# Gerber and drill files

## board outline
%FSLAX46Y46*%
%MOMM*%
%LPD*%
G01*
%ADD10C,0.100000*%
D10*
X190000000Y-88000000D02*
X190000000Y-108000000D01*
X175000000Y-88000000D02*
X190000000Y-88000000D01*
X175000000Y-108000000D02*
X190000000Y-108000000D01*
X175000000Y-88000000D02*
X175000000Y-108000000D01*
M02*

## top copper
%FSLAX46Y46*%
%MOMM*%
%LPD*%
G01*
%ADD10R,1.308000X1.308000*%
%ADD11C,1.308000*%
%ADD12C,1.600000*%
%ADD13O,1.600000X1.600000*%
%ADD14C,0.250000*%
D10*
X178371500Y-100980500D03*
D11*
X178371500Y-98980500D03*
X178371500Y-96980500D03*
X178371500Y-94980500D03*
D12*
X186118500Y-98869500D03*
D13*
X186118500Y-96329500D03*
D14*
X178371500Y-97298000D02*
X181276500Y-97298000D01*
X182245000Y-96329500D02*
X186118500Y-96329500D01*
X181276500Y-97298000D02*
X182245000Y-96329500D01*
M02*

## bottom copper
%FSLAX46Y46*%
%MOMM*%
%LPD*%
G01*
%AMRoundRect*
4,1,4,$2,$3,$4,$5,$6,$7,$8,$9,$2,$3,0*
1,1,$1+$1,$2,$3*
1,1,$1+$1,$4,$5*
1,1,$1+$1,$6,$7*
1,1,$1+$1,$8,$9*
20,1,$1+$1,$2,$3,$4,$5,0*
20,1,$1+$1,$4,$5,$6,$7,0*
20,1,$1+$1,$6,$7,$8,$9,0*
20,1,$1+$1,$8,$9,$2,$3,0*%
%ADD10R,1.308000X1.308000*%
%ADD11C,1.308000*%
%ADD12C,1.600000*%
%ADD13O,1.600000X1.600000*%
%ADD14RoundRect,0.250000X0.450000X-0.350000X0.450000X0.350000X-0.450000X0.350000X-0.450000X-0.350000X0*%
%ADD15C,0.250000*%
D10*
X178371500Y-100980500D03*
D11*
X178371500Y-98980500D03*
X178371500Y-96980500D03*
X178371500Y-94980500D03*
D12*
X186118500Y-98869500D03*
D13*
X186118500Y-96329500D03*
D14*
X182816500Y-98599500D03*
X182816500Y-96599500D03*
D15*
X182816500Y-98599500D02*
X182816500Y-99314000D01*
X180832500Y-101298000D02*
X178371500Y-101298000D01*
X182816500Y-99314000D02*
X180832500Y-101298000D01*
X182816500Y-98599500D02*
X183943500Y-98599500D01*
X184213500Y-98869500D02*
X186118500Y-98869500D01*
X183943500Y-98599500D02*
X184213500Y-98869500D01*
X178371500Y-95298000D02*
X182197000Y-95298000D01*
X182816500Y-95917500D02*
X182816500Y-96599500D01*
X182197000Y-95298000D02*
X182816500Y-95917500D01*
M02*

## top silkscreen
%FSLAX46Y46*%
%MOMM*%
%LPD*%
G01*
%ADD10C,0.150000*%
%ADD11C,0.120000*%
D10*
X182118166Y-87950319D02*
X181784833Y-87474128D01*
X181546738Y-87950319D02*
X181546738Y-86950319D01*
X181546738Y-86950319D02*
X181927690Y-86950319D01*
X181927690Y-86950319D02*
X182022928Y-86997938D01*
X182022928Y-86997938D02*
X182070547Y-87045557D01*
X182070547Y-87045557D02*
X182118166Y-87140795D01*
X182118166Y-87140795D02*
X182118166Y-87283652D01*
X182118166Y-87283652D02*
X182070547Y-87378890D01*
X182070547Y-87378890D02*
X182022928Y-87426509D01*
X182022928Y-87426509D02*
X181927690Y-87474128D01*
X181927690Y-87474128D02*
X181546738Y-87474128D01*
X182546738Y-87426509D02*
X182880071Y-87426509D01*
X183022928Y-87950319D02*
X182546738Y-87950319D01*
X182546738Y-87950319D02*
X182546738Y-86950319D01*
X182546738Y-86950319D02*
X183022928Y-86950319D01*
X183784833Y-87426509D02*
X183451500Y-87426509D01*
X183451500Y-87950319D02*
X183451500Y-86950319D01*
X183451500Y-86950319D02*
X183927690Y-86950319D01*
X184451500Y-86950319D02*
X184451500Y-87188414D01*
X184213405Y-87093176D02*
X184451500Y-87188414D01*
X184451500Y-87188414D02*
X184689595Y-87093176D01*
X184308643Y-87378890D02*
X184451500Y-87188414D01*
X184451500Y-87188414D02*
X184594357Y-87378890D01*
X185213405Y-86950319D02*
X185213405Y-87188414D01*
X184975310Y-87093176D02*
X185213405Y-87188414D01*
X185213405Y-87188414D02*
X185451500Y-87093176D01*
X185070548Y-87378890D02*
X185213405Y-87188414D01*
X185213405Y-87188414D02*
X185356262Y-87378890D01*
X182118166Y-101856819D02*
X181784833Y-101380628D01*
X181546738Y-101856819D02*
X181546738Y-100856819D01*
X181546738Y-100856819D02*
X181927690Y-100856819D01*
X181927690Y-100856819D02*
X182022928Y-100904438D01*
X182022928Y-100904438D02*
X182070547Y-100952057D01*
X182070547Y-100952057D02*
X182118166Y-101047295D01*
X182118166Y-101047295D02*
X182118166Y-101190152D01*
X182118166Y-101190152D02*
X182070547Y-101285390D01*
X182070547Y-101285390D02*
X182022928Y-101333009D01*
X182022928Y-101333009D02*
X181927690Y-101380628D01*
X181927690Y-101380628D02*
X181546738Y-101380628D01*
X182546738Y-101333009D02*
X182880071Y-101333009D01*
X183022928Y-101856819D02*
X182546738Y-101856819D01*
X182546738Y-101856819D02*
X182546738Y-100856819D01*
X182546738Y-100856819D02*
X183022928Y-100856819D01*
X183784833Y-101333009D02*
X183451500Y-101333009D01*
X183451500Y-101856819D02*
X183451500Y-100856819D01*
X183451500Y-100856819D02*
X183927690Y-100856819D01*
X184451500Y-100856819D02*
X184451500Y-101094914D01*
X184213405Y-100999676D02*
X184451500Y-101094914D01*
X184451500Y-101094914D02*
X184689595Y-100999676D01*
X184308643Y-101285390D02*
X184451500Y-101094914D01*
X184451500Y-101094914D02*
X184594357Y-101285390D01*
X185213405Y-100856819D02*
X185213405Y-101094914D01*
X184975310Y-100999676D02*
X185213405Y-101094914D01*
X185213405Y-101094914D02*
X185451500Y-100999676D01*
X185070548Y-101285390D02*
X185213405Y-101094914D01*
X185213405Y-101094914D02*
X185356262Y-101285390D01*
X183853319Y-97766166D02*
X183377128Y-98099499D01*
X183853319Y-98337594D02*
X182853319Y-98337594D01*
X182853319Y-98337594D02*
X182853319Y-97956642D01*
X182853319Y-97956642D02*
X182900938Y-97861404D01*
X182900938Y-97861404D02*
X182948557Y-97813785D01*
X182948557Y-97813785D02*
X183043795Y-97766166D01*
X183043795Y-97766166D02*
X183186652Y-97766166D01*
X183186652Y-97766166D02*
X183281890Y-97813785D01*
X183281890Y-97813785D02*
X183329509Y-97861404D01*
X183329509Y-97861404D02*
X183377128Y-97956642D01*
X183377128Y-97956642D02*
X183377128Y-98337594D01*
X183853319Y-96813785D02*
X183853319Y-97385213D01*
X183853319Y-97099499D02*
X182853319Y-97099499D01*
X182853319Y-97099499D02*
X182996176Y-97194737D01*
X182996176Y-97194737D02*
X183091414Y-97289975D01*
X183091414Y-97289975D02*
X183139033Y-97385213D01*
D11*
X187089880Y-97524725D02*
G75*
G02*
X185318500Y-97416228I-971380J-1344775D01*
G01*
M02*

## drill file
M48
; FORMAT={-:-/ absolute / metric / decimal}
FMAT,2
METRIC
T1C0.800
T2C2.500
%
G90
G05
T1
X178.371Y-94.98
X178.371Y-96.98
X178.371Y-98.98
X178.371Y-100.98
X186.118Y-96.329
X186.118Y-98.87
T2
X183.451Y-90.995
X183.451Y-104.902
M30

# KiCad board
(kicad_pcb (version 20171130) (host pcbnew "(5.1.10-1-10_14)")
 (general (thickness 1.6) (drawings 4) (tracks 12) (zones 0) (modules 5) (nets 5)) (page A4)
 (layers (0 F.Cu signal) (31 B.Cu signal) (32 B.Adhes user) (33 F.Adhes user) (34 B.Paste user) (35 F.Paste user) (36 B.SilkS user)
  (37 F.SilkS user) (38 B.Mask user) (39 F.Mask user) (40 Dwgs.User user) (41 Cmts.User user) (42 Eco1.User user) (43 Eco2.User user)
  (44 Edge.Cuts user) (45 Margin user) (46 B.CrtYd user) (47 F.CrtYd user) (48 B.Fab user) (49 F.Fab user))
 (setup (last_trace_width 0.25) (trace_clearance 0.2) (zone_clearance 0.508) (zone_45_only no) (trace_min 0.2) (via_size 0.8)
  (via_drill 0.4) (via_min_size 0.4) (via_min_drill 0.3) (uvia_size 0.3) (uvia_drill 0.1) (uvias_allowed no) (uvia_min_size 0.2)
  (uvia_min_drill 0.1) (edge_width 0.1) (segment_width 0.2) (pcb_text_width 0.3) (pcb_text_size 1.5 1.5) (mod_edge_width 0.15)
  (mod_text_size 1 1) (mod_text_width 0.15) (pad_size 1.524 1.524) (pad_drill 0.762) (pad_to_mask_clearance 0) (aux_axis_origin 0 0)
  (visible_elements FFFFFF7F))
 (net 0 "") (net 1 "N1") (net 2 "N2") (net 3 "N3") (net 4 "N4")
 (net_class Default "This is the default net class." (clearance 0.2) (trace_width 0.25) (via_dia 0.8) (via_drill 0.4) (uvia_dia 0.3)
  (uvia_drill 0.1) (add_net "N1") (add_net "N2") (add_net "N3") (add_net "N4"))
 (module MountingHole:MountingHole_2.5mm (layer F.Cu) (at 183.4515 90.9955)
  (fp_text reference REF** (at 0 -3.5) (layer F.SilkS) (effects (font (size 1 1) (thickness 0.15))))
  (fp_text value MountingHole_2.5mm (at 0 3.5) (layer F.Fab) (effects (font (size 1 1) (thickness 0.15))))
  (pad 1 np_thru_hole circle (at 0 0) (size 2.5 2.5) (drill 2.5) (layers *.Cu *.Mask)))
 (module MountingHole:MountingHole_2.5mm (layer F.Cu) (at 183.4515 104.902)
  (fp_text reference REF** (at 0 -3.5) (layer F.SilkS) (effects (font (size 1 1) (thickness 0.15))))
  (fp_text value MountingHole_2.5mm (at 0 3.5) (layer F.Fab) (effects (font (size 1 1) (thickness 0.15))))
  (pad 1 np_thru_hole circle (at 0 0) (size 2.5 2.5) (drill 2.5) (layers *.Cu *.Mask)))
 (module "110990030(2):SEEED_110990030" (layer B.Cu) (at 178.3715 97.9805 90)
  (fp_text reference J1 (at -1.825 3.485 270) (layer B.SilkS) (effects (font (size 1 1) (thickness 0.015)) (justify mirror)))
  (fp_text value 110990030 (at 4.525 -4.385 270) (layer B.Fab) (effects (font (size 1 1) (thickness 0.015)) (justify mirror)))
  (pad 1 thru_hole rect (at -3 0 90) (size 1.308 1.308) (drill 0.8) (layers *.Cu *.Mask) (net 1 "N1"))
  (pad 2 thru_hole circle (at -1 0 90) (size 1.308 1.308) (drill 0.8) (layers *.Cu *.Mask) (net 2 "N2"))
  (pad 3 thru_hole circle (at 1 0 90) (size 1.308 1.308) (drill 0.8) (layers *.Cu *.Mask) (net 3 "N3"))
  (pad 4 thru_hole circle (at 3 0 90) (size 1.308 1.308) (drill 0.8) (layers *.Cu *.Mask) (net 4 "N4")))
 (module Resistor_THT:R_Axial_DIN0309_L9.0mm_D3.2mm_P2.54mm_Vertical (layer F.Cu) (at 186.1185 98.8695 90)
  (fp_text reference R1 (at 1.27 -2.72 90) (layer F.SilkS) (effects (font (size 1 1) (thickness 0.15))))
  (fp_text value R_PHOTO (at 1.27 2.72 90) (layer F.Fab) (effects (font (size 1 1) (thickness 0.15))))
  (fp_arc (start 0 0) (end 1.453272 -0.8) (angle -295.326041) (layer F.SilkS) (width 0.12))
  (pad 1 thru_hole circle (at 0 0 90) (size 1.6 1.6) (drill 0.8) (layers *.Cu *.Mask) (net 1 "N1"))
  (pad 2 thru_hole oval (at 2.54 0 90) (size 1.6 1.6) (drill 0.8) (layers *.Cu *.Mask) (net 3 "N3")))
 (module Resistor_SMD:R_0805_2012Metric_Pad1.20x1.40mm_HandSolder (layer B.Cu) (at 182.8165 97.5995 90)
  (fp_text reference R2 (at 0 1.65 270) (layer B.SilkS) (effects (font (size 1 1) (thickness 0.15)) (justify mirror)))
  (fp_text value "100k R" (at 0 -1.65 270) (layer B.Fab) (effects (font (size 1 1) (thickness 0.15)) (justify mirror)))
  (pad 1 smd roundrect (at -1 0 90) (size 1.2 1.4) (layers B.Cu B.Paste B.Mask) (roundrect_rratio 0.208333) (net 1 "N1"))
  (pad 2 smd roundrect (at 1 0 90) (size 1.2 1.4) (layers B.Cu B.Paste B.Mask) (roundrect_rratio 0.208333) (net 4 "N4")))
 (gr_line (start 190 88) (end 190 108) (layer Edge.Cuts) (width 0.1))
 (gr_line (start 175 88) (end 190 88) (layer Edge.Cuts) (width 0.1))
 (gr_line (start 175 108) (end 190 108) (layer Edge.Cuts) (width 0.1))
 (gr_line (start 175 88) (end 175 108) (layer Edge.Cuts) (width 0.1))
 (segment (start 182.8165 98.5995) (end 182.8165 99.314) (width 0.25) (layer B.Cu) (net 1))
 (segment (start 180.8325 101.298) (end 178.3715 101.298) (width 0.25) (layer B.Cu) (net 1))
 (segment (start 182.8165 99.314) (end 180.8325 101.298) (width 0.25) (layer B.Cu) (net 1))
 (segment (start 182.8165 98.5995) (end 183.9435 98.5995) (width 0.25) (layer B.Cu) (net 1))
 (segment (start 184.2135 98.8695) (end 186.1185 98.8695) (width 0.25) (layer B.Cu) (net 1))
 (segment (start 183.9435 98.5995) (end 184.2135 98.8695) (width 0.25) (layer B.Cu) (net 1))
 (segment (start 178.3715 97.298) (end 181.2765 97.298) (width 0.25) (layer F.Cu) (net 3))
 (segment (start 182.245 96.3295) (end 186.1185 96.3295) (width 0.25) (layer F.Cu) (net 3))
 (segment (start 181.2765 97.298) (end 182.245 96.3295) (width 0.25) (layer F.Cu) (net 3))
 (segment (start 178.3715 95.298) (end 182.197 95.298) (width 0.25) (layer B.Cu) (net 4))
 (segment (start 182.8165 95.9175) (end 182.8165 96.5995) (width 0.25) (layer B.Cu) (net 4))
 (segment (start 182.197 95.298) (end 182.8165 95.9175) (width 0.25) (layer B.Cu) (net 4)))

